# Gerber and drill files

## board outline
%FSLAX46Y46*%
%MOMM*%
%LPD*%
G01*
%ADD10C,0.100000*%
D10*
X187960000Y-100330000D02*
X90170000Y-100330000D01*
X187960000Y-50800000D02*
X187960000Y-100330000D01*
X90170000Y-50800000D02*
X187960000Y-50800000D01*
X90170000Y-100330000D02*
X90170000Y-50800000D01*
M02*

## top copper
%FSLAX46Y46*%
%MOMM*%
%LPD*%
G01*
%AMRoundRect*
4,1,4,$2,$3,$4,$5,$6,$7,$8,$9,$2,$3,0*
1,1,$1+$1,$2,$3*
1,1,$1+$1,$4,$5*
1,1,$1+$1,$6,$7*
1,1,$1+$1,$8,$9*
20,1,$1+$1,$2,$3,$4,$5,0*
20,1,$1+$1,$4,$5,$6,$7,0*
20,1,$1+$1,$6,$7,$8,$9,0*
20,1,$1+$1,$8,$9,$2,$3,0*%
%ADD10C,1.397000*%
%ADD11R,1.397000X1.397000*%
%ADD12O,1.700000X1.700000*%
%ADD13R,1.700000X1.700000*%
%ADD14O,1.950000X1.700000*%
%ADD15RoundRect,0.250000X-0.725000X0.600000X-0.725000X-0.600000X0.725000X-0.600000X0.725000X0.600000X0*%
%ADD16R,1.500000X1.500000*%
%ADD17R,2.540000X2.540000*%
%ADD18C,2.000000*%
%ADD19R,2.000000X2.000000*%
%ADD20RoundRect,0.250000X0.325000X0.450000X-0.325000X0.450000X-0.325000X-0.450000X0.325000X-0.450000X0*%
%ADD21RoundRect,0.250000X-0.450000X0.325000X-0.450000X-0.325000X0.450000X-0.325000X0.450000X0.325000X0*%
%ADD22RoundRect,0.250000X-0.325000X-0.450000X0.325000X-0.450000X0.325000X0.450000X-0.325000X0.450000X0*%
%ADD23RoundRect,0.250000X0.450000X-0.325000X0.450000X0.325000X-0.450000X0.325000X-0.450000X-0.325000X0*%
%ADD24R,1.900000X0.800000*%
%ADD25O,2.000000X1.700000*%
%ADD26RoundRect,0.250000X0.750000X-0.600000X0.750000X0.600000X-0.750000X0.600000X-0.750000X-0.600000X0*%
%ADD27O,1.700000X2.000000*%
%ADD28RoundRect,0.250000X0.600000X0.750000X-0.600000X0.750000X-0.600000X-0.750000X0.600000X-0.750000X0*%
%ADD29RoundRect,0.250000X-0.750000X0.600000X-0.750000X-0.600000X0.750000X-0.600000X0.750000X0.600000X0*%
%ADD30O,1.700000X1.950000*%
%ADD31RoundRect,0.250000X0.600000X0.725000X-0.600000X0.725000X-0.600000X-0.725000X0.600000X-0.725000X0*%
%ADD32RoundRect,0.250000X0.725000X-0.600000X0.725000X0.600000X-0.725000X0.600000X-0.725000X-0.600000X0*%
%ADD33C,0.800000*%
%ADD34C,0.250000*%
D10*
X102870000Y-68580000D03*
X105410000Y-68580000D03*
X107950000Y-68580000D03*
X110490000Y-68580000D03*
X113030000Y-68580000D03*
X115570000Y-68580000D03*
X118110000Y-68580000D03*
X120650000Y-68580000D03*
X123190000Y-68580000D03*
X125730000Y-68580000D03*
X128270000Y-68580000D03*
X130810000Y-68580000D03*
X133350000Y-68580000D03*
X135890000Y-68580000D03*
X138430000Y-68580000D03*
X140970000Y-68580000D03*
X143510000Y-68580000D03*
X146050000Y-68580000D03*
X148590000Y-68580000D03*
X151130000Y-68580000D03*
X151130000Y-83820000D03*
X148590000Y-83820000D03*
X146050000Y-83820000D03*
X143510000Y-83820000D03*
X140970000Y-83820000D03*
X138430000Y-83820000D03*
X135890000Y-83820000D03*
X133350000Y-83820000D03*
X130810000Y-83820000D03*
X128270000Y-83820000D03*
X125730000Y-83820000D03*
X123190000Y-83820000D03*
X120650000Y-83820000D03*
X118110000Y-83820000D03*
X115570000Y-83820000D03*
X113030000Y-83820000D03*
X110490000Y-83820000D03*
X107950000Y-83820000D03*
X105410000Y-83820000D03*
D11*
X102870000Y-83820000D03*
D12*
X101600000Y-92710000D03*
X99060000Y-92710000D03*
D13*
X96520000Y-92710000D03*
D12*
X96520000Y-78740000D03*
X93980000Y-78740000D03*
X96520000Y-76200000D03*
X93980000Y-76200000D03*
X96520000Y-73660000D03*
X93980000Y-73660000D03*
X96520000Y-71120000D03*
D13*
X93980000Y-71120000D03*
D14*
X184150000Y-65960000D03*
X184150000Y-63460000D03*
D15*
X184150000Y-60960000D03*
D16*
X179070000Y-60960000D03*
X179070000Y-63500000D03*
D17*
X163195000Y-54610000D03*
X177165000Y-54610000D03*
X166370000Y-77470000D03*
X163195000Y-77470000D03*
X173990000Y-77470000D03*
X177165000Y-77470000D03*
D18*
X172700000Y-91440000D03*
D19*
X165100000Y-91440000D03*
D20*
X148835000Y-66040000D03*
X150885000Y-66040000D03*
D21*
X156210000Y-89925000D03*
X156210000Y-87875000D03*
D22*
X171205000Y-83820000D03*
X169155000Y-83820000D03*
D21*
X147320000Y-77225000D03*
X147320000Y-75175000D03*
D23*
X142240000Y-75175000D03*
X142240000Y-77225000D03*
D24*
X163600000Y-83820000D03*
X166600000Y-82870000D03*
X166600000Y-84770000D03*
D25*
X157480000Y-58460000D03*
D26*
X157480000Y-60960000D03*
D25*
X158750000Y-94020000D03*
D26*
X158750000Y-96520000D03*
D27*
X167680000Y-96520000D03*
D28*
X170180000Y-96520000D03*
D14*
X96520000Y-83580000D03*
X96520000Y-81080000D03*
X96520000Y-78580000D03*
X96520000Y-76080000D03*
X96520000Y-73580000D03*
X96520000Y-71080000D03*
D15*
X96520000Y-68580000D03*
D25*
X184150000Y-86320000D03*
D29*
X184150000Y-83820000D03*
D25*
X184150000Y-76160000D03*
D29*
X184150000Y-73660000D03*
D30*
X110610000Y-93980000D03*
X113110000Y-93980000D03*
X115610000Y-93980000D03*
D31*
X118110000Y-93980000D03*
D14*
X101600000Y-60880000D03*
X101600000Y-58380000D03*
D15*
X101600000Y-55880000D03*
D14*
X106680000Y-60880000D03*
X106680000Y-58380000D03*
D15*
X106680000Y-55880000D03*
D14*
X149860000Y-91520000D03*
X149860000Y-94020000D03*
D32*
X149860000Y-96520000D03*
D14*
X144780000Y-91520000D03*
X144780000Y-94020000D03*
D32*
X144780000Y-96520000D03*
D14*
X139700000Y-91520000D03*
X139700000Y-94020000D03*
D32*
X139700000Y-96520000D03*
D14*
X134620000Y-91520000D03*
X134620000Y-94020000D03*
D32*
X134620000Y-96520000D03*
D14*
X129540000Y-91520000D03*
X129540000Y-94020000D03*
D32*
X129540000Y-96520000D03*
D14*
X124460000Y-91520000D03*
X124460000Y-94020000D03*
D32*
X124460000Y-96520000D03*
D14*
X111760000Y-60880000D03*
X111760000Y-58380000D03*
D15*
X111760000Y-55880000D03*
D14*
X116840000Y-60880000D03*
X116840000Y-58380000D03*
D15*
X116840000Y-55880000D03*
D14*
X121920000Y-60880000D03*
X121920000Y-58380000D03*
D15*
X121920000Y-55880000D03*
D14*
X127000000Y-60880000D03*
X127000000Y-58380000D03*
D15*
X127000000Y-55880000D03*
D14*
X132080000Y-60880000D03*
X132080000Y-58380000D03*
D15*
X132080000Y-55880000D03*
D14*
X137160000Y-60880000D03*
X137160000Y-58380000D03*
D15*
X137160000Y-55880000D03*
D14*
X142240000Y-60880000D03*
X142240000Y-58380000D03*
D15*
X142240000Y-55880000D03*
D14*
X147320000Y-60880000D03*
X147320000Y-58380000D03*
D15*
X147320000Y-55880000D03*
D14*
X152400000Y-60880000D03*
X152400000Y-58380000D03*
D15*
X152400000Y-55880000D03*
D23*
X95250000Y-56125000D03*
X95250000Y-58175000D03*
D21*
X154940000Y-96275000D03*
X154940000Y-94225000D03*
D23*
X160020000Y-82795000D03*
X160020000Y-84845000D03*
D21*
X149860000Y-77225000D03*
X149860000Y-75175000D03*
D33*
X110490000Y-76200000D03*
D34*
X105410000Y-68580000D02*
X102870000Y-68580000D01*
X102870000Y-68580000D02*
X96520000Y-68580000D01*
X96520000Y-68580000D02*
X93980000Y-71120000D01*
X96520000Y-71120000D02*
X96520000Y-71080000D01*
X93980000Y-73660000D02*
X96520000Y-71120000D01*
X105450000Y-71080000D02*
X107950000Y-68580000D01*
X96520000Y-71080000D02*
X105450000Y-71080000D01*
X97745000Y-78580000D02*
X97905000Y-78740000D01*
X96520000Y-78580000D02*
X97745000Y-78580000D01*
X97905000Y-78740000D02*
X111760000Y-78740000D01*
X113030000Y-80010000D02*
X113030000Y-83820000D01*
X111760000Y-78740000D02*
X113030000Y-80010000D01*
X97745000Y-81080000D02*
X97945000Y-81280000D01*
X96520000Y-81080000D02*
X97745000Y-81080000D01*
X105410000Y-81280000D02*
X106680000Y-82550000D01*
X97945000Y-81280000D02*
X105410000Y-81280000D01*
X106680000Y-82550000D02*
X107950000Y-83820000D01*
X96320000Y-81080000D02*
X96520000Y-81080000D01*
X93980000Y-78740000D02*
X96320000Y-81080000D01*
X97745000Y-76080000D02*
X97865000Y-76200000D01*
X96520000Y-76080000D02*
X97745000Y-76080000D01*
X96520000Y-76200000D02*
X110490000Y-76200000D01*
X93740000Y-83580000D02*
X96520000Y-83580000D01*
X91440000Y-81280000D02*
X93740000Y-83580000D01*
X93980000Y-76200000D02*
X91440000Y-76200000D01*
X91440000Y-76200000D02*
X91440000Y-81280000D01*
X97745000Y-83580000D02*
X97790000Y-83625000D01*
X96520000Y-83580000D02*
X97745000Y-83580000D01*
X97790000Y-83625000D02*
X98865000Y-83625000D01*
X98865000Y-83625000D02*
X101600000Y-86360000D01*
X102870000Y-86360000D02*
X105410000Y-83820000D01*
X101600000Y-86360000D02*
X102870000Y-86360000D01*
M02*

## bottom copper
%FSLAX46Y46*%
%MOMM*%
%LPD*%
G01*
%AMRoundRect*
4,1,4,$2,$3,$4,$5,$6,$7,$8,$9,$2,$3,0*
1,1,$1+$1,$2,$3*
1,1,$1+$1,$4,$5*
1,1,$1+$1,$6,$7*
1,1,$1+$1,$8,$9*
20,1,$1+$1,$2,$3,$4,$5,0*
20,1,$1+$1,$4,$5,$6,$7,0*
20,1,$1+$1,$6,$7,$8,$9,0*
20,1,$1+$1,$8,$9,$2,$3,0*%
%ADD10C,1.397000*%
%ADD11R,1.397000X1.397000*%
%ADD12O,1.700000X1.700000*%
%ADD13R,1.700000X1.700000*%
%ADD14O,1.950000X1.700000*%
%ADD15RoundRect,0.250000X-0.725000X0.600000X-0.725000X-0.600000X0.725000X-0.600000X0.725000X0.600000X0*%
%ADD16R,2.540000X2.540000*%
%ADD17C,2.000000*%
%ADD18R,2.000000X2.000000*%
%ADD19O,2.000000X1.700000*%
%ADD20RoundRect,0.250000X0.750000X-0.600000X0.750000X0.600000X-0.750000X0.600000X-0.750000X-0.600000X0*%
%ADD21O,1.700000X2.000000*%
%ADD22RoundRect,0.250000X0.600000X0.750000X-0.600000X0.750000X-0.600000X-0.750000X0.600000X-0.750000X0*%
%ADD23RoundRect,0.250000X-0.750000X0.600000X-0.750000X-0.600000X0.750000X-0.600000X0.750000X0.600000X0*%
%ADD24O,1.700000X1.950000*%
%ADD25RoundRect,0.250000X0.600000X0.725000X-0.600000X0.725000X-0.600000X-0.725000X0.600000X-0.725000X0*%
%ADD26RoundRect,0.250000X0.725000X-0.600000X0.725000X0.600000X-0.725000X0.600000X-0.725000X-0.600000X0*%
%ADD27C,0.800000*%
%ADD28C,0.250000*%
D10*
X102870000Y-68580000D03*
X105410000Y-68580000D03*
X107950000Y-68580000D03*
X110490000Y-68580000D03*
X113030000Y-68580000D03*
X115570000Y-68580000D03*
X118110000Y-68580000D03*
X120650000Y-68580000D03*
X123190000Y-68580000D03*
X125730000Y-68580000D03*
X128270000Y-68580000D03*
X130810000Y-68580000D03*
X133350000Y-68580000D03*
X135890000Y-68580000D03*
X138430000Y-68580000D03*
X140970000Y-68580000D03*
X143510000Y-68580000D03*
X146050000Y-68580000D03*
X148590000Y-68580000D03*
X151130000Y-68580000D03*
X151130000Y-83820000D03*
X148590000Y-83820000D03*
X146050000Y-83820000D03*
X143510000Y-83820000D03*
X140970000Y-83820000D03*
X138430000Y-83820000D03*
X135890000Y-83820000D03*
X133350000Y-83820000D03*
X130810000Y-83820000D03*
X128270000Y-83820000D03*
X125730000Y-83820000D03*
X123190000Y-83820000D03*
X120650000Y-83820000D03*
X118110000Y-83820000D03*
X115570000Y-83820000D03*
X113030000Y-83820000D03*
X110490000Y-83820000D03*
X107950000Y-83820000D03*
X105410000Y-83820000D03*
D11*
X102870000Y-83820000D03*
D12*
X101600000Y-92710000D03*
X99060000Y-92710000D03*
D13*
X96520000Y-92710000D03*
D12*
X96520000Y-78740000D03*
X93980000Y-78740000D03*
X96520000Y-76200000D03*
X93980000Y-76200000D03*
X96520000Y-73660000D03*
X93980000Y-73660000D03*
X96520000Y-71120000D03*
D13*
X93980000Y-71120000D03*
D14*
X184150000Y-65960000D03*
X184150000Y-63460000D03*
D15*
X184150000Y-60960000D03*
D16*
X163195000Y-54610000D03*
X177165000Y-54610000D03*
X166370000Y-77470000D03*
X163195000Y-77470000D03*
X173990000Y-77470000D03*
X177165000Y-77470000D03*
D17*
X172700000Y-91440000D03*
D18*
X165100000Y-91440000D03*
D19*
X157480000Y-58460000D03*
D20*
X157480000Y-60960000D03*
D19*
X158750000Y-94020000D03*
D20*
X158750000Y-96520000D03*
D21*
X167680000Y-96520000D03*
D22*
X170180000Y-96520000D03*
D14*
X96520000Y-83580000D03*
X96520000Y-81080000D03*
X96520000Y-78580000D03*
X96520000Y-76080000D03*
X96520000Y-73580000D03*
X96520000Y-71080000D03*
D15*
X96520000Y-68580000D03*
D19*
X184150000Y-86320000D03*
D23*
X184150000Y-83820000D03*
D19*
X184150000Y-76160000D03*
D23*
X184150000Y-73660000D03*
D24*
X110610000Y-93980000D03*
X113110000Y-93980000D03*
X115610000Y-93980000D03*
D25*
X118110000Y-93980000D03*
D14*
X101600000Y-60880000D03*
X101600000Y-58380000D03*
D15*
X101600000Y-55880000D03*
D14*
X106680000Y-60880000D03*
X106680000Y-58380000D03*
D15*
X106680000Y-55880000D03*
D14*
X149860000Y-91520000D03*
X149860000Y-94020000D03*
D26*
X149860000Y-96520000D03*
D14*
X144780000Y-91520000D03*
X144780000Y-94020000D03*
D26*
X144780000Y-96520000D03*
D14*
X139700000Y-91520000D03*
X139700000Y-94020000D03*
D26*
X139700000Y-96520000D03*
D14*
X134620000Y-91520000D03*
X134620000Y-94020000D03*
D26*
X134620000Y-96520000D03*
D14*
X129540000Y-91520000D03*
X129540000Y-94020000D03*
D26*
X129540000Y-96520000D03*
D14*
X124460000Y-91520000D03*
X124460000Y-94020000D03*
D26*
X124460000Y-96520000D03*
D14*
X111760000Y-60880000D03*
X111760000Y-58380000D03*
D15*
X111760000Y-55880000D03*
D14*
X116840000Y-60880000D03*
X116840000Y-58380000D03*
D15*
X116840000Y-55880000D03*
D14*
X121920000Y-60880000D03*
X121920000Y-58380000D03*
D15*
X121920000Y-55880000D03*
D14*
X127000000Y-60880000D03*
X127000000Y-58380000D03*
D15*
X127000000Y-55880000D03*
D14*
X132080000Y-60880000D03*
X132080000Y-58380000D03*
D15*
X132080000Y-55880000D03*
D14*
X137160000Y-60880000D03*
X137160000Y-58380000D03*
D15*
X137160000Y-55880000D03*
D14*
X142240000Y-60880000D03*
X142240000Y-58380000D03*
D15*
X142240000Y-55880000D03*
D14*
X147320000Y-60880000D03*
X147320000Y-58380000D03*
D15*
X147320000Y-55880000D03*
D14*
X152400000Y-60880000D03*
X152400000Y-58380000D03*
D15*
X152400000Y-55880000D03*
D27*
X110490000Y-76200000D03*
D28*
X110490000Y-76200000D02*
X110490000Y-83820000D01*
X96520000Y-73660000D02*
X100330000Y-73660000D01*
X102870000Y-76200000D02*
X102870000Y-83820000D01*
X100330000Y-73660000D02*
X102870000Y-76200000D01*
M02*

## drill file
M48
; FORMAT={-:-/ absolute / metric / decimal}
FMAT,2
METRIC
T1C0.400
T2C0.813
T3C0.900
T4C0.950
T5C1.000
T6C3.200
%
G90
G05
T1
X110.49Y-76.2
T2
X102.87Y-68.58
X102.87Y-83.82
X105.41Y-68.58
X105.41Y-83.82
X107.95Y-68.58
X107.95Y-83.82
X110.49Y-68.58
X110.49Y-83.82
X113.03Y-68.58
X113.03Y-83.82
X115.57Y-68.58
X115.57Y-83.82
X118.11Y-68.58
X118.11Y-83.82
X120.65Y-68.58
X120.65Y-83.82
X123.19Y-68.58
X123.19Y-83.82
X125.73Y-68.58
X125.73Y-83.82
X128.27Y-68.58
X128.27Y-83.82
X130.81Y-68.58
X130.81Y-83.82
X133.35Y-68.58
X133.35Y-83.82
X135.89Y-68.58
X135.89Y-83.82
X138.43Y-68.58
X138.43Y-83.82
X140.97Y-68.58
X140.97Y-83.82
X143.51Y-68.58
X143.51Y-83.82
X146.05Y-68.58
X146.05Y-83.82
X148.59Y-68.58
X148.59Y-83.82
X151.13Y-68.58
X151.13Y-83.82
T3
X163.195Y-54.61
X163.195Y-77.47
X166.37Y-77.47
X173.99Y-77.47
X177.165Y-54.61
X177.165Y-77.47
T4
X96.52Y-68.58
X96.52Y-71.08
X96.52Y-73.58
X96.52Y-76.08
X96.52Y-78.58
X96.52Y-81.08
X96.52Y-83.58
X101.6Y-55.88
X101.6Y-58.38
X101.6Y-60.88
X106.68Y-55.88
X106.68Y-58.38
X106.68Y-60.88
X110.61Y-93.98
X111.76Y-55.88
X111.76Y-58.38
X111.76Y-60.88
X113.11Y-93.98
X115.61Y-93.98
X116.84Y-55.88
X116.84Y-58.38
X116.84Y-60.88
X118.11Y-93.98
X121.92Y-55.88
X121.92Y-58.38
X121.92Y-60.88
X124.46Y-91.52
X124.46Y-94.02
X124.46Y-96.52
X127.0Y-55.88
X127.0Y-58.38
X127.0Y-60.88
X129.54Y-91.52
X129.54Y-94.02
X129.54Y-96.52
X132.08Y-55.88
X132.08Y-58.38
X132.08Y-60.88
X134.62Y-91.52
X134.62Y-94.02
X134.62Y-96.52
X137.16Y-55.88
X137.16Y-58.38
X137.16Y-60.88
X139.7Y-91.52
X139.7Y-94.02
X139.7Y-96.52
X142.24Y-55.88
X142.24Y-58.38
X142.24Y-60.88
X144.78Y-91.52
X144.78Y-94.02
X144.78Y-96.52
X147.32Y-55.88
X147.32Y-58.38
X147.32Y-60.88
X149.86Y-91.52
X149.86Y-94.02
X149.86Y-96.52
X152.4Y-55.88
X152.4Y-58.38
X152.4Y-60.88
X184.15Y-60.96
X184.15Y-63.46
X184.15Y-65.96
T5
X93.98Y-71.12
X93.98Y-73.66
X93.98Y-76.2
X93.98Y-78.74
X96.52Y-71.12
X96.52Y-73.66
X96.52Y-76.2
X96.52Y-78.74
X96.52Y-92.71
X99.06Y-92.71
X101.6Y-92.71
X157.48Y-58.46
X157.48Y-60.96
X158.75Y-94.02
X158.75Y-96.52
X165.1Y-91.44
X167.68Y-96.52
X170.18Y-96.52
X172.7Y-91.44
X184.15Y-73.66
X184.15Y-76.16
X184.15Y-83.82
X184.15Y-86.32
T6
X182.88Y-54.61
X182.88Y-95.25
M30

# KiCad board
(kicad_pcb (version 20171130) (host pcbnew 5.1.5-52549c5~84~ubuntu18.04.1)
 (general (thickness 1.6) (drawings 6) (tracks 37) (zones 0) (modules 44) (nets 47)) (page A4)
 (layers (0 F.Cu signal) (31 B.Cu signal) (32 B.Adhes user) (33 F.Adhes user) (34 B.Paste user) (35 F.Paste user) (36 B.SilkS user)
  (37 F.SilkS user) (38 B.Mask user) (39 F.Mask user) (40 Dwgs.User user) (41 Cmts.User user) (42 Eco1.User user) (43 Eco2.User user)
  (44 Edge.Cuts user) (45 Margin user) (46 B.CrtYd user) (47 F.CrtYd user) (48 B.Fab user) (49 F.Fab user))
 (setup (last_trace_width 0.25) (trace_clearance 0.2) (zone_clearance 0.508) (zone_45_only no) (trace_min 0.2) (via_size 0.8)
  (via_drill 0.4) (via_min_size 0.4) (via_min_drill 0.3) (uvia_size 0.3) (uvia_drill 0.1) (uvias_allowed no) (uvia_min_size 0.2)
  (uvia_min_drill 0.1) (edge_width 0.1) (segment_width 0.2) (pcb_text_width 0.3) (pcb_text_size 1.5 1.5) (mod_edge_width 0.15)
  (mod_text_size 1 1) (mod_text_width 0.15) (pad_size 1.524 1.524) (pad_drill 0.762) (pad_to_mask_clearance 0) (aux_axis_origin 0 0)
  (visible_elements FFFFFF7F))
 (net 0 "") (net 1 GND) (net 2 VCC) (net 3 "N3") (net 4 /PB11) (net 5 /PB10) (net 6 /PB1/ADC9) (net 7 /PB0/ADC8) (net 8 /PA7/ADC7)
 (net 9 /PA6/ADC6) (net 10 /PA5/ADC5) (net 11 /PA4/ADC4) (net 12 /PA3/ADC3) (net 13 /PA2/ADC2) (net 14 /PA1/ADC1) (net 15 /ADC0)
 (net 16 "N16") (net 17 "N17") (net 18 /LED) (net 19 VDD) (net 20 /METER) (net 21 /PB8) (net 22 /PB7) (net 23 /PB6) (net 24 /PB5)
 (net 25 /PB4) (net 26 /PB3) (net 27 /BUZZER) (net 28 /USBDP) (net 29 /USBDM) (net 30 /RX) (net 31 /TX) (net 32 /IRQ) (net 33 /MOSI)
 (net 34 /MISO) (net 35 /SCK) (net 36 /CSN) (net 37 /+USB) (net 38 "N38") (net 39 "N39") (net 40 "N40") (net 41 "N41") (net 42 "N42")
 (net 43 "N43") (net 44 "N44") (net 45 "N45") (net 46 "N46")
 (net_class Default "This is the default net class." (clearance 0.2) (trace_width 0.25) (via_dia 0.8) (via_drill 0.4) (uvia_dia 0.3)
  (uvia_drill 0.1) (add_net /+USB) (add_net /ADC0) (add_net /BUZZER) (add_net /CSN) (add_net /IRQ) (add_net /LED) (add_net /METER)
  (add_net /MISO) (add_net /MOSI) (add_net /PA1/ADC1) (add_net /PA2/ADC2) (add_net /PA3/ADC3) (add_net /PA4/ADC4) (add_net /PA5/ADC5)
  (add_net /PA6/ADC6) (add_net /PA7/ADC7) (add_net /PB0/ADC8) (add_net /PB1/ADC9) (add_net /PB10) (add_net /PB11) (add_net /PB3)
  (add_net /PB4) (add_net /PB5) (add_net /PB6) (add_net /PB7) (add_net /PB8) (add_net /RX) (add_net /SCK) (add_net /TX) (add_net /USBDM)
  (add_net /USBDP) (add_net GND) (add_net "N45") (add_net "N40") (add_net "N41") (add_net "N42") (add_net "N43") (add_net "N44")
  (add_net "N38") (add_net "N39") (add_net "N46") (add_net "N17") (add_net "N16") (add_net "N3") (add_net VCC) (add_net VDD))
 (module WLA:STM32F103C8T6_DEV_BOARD (layer F.Cu) (at 127 76.2)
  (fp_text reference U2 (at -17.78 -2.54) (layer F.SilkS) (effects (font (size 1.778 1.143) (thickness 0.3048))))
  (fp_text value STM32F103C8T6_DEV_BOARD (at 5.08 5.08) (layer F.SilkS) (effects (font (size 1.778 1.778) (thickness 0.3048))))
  (pad 40 thru_hole circle (at -24.13 -7.62) (size 1.397 1.397) (drill 0.8128) (layers *.Cu *.Mask) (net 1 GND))
  (pad 39 thru_hole circle (at -21.59 -7.62) (size 1.397 1.397) (drill 0.8128) (layers *.Cu *.Mask) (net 1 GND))
  (pad 38 thru_hole circle (at -19.05 -7.62) (size 1.397 1.397) (drill 0.8128) (layers *.Cu *.Mask) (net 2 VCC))
  (pad 37 thru_hole circle (at -16.51 -7.62) (size 1.397 1.397) (drill 0.8128) (layers *.Cu *.Mask) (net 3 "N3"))
  (pad 36 thru_hole circle (at -13.97 -7.62) (size 1.397 1.397) (drill 0.8128) (layers *.Cu *.Mask) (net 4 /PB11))
  (pad 35 thru_hole circle (at -11.43 -7.62) (size 1.397 1.397) (drill 0.8128) (layers *.Cu *.Mask) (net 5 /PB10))
  (pad 34 thru_hole circle (at -8.89 -7.62) (size 1.397 1.397) (drill 0.8128) (layers *.Cu *.Mask) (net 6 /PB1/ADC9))
  (pad 33 thru_hole circle (at -6.35 -7.62) (size 1.397 1.397) (drill 0.8128) (layers *.Cu *.Mask) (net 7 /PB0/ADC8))
  (pad 32 thru_hole circle (at -3.81 -7.62) (size 1.397 1.397) (drill 0.8128) (layers *.Cu *.Mask) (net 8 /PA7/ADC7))
  (pad 31 thru_hole circle (at -1.27 -7.62) (size 1.397 1.397) (drill 0.8128) (layers *.Cu *.Mask) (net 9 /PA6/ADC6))
  (pad 30 thru_hole circle (at 1.27 -7.62) (size 1.397 1.397) (drill 0.8128) (layers *.Cu *.Mask) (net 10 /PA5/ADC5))
  (pad 29 thru_hole circle (at 3.81 -7.62) (size 1.397 1.397) (drill 0.8128) (layers *.Cu *.Mask) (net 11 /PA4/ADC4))
  (pad 28 thru_hole circle (at 6.35 -7.62) (size 1.397 1.397) (drill 0.8128) (layers *.Cu *.Mask) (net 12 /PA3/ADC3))
  (pad 27 thru_hole circle (at 8.89 -7.62) (size 1.397 1.397) (drill 0.8128) (layers *.Cu *.Mask) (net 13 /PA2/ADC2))
  (pad 26 thru_hole circle (at 11.43 -7.62) (size 1.397 1.397) (drill 0.8128) (layers *.Cu *.Mask) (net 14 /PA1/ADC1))
  (pad 25 thru_hole circle (at 13.97 -7.62) (size 1.397 1.397) (drill 0.8128) (layers *.Cu *.Mask) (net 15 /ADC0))
  (pad 24 thru_hole circle (at 16.51 -7.62) (size 1.397 1.397) (drill 0.8128) (layers *.Cu *.Mask) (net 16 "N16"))
  (pad 23 thru_hole circle (at 19.05 -7.62) (size 1.397 1.397) (drill 0.8128) (layers *.Cu *.Mask) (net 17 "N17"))
  (pad 22 thru_hole circle (at 21.59 -7.62) (size 1.397 1.397) (drill 0.8128) (layers *.Cu *.Mask) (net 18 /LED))
  (pad 21 thru_hole circle (at 24.13 -7.62) (size 1.397 1.397) (drill 0.8128) (layers *.Cu *.Mask) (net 2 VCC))
  (pad 20 thru_hole circle (at 24.13 7.62) (size 1.397 1.397) (drill 0.8128) (layers *.Cu *.Mask) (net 2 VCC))
  (pad 19 thru_hole circle (at 21.59 7.62) (size 1.397 1.397) (drill 0.8128) (layers *.Cu *.Mask) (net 1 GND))
  (pad 18 thru_hole circle (at 19.05 7.62) (size 1.397 1.397) (drill 0.8128) (layers *.Cu *.Mask) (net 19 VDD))
  (pad 17 thru_hole circle (at 16.51 7.62) (size 1.397 1.397) (drill 0.8128) (layers *.Cu *.Mask) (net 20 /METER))
  (pad 16 thru_hole circle (at 13.97 7.62) (size 1.397 1.397) (drill 0.8128) (layers *.Cu *.Mask) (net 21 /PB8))
  (pad 15 thru_hole circle (at 11.43 7.62) (size 1.397 1.397) (drill 0.8128) (layers *.Cu *.Mask) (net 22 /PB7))
  (pad 14 thru_hole circle (at 8.89 7.62) (size 1.397 1.397) (drill 0.8128) (layers *.Cu *.Mask) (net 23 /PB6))
  (pad 13 thru_hole circle (at 6.35 7.62) (size 1.397 1.397) (drill 0.8128) (layers *.Cu *.Mask) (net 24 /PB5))
  (pad 12 thru_hole circle (at 3.81 7.62) (size 1.397 1.397) (drill 0.8128) (layers *.Cu *.Mask) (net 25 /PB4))
  (pad 11 thru_hole circle (at 1.27 7.62) (size 1.397 1.397) (drill 0.8128) (layers *.Cu *.Mask) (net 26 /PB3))
  (pad 10 thru_hole circle (at -1.27 7.62) (size 1.397 1.397) (drill 0.8128) (layers *.Cu *.Mask) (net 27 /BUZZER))
  (pad 9 thru_hole circle (at -3.81 7.62) (size 1.397 1.397) (drill 0.8128) (layers *.Cu *.Mask) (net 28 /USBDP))
  (pad 8 thru_hole circle (at -6.35 7.62) (size 1.397 1.397) (drill 0.8128) (layers *.Cu *.Mask) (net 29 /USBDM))
  (pad 7 thru_hole circle (at -8.89 7.62) (size 1.397 1.397) (drill 0.8128) (layers *.Cu *.Mask) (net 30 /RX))
  (pad 6 thru_hole circle (at -11.43 7.62) (size 1.397 1.397) (drill 0.8128) (layers *.Cu *.Mask) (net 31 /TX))
  (pad 5 thru_hole circle (at -13.97 7.62) (size 1.397 1.397) (drill 0.8128) (layers *.Cu *.Mask) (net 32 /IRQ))
  (pad 4 thru_hole circle (at -16.51 7.62) (size 1.397 1.397) (drill 0.8128) (layers *.Cu *.Mask) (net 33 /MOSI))
  (pad 3 thru_hole circle (at -19.05 7.62) (size 1.397 1.397) (drill 0.8128) (layers *.Cu *.Mask) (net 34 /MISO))
  (pad 2 thru_hole circle (at -21.59 7.62) (size 1.397 1.397) (drill 0.8128) (layers *.Cu *.Mask) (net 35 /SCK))
  (pad 1 thru_hole rect (at -24.13 7.62) (size 1.397 1.397) (drill 0.8128) (layers *.Cu *.Mask) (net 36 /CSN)))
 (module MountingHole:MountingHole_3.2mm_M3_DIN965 (layer F.Cu) (at 182.88 95.25)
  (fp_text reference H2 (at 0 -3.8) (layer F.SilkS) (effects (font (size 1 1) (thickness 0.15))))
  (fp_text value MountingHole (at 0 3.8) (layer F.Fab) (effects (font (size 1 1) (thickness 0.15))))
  (pad 1 np_thru_hole circle (at 0 0) (size 3.2 3.2) (drill 3.2) (layers *.Cu *.Mask)))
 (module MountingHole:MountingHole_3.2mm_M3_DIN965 (layer F.Cu) (at 182.88 54.61)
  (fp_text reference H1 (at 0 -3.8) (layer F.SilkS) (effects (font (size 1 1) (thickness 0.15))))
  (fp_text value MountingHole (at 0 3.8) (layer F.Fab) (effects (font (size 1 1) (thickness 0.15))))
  (pad 1 np_thru_hole circle (at 0 0) (size 3.2 3.2) (drill 3.2) (layers *.Cu *.Mask)))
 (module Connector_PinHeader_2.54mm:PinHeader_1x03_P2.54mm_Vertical (layer F.Cu) (at 96.52 92.71 90)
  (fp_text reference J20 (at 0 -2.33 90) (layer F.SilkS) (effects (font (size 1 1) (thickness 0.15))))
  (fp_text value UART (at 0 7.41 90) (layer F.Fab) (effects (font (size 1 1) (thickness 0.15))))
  (pad 3 thru_hole oval (at 0 5.08 90) (size 1.7 1.7) (drill 1) (layers *.Cu *.Mask) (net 30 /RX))
  (pad 2 thru_hole oval (at 0 2.54 90) (size 1.7 1.7) (drill 1) (layers *.Cu *.Mask) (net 31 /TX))
  (pad 1 thru_hole rect (at 0 0 90) (size 1.7 1.7) (drill 1) (layers *.Cu *.Mask) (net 1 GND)))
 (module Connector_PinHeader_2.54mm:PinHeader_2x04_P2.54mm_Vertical (layer F.Cu) (at 93.98 71.12)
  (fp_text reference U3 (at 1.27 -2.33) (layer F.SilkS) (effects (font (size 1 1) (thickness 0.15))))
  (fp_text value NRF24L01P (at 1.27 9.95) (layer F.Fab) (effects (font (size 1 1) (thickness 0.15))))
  (pad 8 thru_hole oval (at 2.54 7.62) (size 1.7 1.7) (drill 1) (layers *.Cu *.Mask) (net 32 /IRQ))
  (pad 7 thru_hole oval (at 0 7.62) (size 1.7 1.7) (drill 1) (layers *.Cu *.Mask) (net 34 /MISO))
  (pad 6 thru_hole oval (at 2.54 5.08) (size 1.7 1.7) (drill 1) (layers *.Cu *.Mask) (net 33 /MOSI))
  (pad 5 thru_hole oval (at 0 5.08) (size 1.7 1.7) (drill 1) (layers *.Cu *.Mask) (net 35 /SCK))
  (pad 4 thru_hole oval (at 2.54 2.54) (size 1.7 1.7) (drill 1) (layers *.Cu *.Mask) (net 36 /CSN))
  (pad 3 thru_hole oval (at 0 2.54) (size 1.7 1.7) (drill 1) (layers *.Cu *.Mask) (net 2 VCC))
  (pad 2 thru_hole oval (at 2.54 0) (size 1.7 1.7) (drill 1) (layers *.Cu *.Mask) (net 2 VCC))
  (pad 1 thru_hole rect (at 0 0) (size 1.7 1.7) (drill 1) (layers *.Cu *.Mask) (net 1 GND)))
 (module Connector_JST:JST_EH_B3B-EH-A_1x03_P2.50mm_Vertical (layer F.Cu) (at 184.15 60.96 270)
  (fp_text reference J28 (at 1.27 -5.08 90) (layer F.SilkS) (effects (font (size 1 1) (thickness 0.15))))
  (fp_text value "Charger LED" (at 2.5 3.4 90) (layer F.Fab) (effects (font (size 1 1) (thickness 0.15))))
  (pad 3 thru_hole oval (at 5 0 270) (size 1.7 1.95) (drill 0.95) (layers *.Cu *.Mask) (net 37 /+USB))
  (pad 2 thru_hole oval (at 2.5 0 270) (size 1.7 1.95) (drill 0.95) (layers *.Cu *.Mask) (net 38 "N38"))
  (pad 1 thru_hole roundrect (at 0 0 270) (size 1.7 1.95) (drill 0.95) (layers *.Cu *.Mask) (roundrect_rratio 0.147059) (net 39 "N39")))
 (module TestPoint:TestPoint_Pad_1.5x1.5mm (layer F.Cu) (at 179.07 60.96 90)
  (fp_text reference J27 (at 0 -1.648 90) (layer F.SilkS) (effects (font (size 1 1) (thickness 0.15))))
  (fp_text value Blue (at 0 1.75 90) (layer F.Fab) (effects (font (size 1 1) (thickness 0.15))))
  (pad 1 smd rect (at 0 0 90) (size 1.5 1.5) (layers F.Cu F.Mask) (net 39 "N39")))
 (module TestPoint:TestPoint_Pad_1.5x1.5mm (layer F.Cu) (at 179.07 63.5 90)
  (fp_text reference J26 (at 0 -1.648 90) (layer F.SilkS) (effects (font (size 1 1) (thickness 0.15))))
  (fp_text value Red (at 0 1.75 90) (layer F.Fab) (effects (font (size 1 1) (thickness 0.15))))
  (pad 1 smd rect (at 0 0 90) (size 1.5 1.5) (layers F.Cu F.Mask) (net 38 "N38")))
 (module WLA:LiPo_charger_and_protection (layer F.Cu) (at 170.18 66.04 270)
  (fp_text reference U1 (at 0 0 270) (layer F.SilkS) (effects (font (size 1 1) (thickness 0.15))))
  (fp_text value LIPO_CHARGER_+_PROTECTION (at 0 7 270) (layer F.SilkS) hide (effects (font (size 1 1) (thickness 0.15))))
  (pad 6 thru_hole rect (at -11.43 6.985 270) (size 2.54 2.54) (drill 0.9) (layers *.Cu *.Mask) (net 1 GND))
  (pad 5 thru_hole rect (at -11.43 -6.985 270) (size 2.54 2.54) (drill 0.9) (layers *.Cu *.Mask) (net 37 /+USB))
  (pad 2 thru_hole rect (at 11.43 3.81 270) (size 2.54 2.54) (drill 0.9) (layers *.Cu *.Mask) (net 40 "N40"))
  (pad 4 thru_hole rect (at 11.43 6.985 270) (size 2.54 2.54) (drill 0.9) (layers *.Cu *.Mask) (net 1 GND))
  (pad 1 thru_hole rect (at 11.43 -3.81 270) (size 2.54 2.54) (drill 0.9) (layers *.Cu *.Mask) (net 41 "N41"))
  (pad 3 thru_hole rect (at 11.43 -6.985 270) (size 2.54 2.54) (drill 0.9) (layers *.Cu *.Mask) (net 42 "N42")))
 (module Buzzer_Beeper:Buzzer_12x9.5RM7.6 (layer F.Cu) (at 165.1 91.44)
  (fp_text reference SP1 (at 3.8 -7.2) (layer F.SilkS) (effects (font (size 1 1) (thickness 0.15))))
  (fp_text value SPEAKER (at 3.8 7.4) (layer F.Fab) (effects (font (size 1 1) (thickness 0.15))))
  (pad 2 thru_hole circle (at 7.6 0) (size 2 2) (drill 1) (layers *.Cu *.Mask) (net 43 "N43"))
  (pad 1 thru_hole rect (at 0 0) (size 2 2) (drill 1) (layers *.Cu *.Mask) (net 19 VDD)))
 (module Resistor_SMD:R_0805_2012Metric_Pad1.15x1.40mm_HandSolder (layer F.Cu) (at 149.86 66.04 180)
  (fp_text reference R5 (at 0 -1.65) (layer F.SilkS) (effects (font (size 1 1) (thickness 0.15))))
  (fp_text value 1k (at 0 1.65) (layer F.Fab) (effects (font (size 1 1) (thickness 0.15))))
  (pad 2 smd roundrect (at 1.025 0 180) (size 1.15 1.4) (layers F.Cu F.Paste F.Mask) (roundrect_rratio 0.217391) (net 18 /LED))
  (pad 1 smd roundrect (at -1.025 0 180) (size 1.15 1.4) (layers F.Cu F.Paste F.Mask) (roundrect_rratio 0.217391) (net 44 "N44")))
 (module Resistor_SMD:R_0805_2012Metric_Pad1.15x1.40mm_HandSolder (layer F.Cu) (at 156.21 88.9 270)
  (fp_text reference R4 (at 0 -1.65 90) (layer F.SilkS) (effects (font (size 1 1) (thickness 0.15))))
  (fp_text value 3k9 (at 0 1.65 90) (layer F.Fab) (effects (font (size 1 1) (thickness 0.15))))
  (pad 2 smd roundrect (at 1.025 0 270) (size 1.15 1.4) (layers F.Cu F.Paste F.Mask) (roundrect_rratio 0.217391) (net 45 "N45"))
  (pad 1 smd roundrect (at -1.025 0 270) (size 1.15 1.4) (layers F.Cu F.Paste F.Mask) (roundrect_rratio 0.217391) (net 20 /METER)))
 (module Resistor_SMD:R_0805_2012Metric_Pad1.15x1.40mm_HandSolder (layer F.Cu) (at 170.18 83.82)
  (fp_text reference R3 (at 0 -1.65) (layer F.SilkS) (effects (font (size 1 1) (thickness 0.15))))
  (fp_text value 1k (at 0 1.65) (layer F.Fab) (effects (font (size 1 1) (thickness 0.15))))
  (pad 2 smd roundrect (at 1.025 0) (size 1.15 1.4) (layers F.Cu F.Paste F.Mask) (roundrect_rratio 0.217391) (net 27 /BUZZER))
  (pad 1 smd roundrect (at -1.025 0) (size 1.15 1.4) (layers F.Cu F.Paste F.Mask) (roundrect_rratio 0.217391) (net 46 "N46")))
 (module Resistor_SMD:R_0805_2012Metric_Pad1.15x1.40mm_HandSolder (layer F.Cu) (at 147.32 76.2 270)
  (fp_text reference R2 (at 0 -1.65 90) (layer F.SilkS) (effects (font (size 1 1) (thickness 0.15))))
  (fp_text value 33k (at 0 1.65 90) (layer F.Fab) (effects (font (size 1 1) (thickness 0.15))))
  (pad 2 smd roundrect (at 1.025 0 270) (size 1.15 1.4) (layers F.Cu F.Paste F.Mask) (roundrect_rratio 0.217391) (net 1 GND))
  (pad 1 smd roundrect (at -1.025 0 270) (size 1.15 1.4) (layers F.Cu F.Paste F.Mask) (roundrect_rratio 0.217391) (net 15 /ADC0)))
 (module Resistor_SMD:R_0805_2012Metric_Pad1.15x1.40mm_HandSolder (layer F.Cu) (at 142.24 76.2 90)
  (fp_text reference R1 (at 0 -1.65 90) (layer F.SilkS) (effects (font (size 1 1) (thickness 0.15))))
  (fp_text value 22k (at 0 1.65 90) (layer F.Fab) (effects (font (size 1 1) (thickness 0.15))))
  (pad 2 smd roundrect (at 1.025 0 90) (size 1.15 1.4) (layers F.Cu F.Paste F.Mask) (roundrect_rratio 0.217391) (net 15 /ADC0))
  (pad 1 smd roundrect (at -1.025 0 90) (size 1.15 1.4) (layers F.Cu F.Paste F.Mask) (roundrect_rratio 0.217391) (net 19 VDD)))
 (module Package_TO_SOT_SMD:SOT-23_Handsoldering (layer F.Cu) (at 165.1 83.82 180)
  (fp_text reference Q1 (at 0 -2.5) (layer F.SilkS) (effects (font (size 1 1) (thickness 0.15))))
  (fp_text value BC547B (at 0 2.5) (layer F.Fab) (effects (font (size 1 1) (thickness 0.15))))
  (pad 3 smd rect (at 1.5 0 180) (size 1.9 0.8) (layers F.Cu F.Paste F.Mask) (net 1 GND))
  (pad 2 smd rect (at -1.5 0.95 180) (size 1.9 0.8) (layers F.Cu F.Paste F.Mask) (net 46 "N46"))
  (pad 1 smd rect (at -1.5 -0.95 180) (size 1.9 0.8) (layers F.Cu F.Paste F.Mask) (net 43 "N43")))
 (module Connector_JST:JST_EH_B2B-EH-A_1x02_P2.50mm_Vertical (layer F.Cu) (at 157.48 60.96 90)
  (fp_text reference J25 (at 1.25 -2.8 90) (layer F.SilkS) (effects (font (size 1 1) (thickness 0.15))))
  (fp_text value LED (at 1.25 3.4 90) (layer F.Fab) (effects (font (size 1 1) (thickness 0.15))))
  (pad 2 thru_hole oval (at 2.5 0 90) (size 1.7 2) (drill 1) (layers *.Cu *.Mask) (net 2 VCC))
  (pad 1 thru_hole roundrect (at 0 0 90) (size 1.7 2) (drill 1) (layers *.Cu *.Mask) (roundrect_rratio 0.147059) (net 44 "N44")))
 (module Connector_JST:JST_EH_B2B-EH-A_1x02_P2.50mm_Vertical (layer F.Cu) (at 158.75 96.52 90)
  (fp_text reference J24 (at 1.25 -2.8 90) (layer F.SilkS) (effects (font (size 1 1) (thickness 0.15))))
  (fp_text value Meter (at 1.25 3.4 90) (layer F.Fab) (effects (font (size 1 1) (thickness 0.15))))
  (pad 2 thru_hole oval (at 2.5 0 90) (size 1.7 2) (drill 1) (layers *.Cu *.Mask) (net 45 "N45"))
  (pad 1 thru_hole roundrect (at 0 0 90) (size 1.7 2) (drill 1) (layers *.Cu *.Mask) (roundrect_rratio 0.147059) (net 1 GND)))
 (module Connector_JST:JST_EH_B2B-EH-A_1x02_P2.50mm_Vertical (layer F.Cu) (at 170.18 96.52 180)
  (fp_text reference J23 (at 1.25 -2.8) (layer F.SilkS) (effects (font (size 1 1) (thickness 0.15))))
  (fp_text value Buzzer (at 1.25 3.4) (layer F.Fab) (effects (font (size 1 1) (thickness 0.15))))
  (pad 2 thru_hole oval (at 2.5 0 180) (size 1.7 2) (drill 1) (layers *.Cu *.Mask) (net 19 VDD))
  (pad 1 thru_hole roundrect (at 0 0 180) (size 1.7 2) (drill 1) (layers *.Cu *.Mask) (roundrect_rratio 0.147059) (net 43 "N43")))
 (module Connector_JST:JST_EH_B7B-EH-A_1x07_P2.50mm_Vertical (layer F.Cu) (at 96.52 68.58 270)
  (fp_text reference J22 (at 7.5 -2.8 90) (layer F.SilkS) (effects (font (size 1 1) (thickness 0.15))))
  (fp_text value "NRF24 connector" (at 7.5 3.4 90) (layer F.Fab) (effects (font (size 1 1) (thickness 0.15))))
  (pad 7 thru_hole oval (at 15 0 270) (size 1.7 1.95) (drill 0.95) (layers *.Cu *.Mask) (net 35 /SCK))
  (pad 6 thru_hole oval (at 12.5 0 270) (size 1.7 1.95) (drill 0.95) (layers *.Cu *.Mask) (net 34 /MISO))
  (pad 5 thru_hole oval (at 10 0 270) (size 1.7 1.95) (drill 0.95) (layers *.Cu *.Mask) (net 32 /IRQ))
  (pad 4 thru_hole oval (at 7.5 0 270) (size 1.7 1.95) (drill 0.95) (layers *.Cu *.Mask) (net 33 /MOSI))
  (pad 3 thru_hole oval (at 5 0 270) (size 1.7 1.95) (drill 0.95) (layers *.Cu *.Mask) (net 36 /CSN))
  (pad 2 thru_hole oval (at 2.5 0 270) (size 1.7 1.95) (drill 0.95) (layers *.Cu *.Mask) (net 2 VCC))
  (pad 1 thru_hole roundrect (at 0 0 270) (size 1.7 1.95) (drill 0.95) (layers *.Cu *.Mask) (roundrect_rratio 0.147059) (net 1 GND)))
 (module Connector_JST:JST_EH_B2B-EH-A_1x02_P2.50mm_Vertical (layer F.Cu) (at 184.15 83.82 270)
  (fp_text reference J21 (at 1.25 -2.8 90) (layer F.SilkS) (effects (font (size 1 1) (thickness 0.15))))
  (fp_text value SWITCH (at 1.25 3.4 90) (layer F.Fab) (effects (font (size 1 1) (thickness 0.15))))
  (pad 2 thru_hole oval (at 2.5 0 270) (size 1.7 2) (drill 1) (layers *.Cu *.Mask) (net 19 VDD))
  (pad 1 thru_hole roundrect (at 0 0 270) (size 1.7 2) (drill 1) (layers *.Cu *.Mask) (roundrect_rratio 0.147059) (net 42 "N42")))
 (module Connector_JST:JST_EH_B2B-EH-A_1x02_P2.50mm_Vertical (layer F.Cu) (at 184.15 73.66 270)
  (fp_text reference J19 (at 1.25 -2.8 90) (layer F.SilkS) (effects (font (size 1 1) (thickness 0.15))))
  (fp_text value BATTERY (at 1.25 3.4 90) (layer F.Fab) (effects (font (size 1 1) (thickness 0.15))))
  (pad 2 thru_hole oval (at 2.5 0 270) (size 1.7 2) (drill 1) (layers *.Cu *.Mask) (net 41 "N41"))
  (pad 1 thru_hole roundrect (at 0 0 270) (size 1.7 2) (drill 1) (layers *.Cu *.Mask) (roundrect_rratio 0.147059) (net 40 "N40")))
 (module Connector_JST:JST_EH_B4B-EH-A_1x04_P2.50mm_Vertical (layer F.Cu) (at 118.11 93.98 180)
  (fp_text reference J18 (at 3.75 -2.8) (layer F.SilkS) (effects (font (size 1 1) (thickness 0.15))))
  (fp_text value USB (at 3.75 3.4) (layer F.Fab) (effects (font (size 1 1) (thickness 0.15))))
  (pad 4 thru_hole oval (at 7.5 0 180) (size 1.7 1.95) (drill 0.95) (layers *.Cu *.Mask) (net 37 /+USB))
  (pad 3 thru_hole oval (at 5 0 180) (size 1.7 1.95) (drill 0.95) (layers *.Cu *.Mask) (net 29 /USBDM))
  (pad 2 thru_hole oval (at 2.5 0 180) (size 1.7 1.95) (drill 0.95) (layers *.Cu *.Mask) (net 28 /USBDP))
  (pad 1 thru_hole roundrect (at 0 0 180) (size 1.7 1.95) (drill 0.95) (layers *.Cu *.Mask) (roundrect_rratio 0.147059) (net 1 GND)))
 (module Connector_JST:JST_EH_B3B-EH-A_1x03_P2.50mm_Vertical (layer F.Cu) (at 101.6 55.88 270)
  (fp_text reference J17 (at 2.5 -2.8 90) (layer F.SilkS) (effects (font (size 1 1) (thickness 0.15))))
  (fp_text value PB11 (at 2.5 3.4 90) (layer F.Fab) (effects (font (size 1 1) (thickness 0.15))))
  (pad 3 thru_hole oval (at 5 0 270) (size 1.7 1.95) (drill 0.95) (layers *.Cu *.Mask) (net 4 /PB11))
  (pad 2 thru_hole oval (at 2.5 0 270) (size 1.7 1.95) (drill 0.95) (layers *.Cu *.Mask) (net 2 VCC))
  (pad 1 thru_hole roundrect (at 0 0 270) (size 1.7 1.95) (drill 0.95) (layers *.Cu *.Mask) (roundrect_rratio 0.147059) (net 1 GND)))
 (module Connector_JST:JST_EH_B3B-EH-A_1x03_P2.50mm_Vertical (layer F.Cu) (at 106.68 55.88 270)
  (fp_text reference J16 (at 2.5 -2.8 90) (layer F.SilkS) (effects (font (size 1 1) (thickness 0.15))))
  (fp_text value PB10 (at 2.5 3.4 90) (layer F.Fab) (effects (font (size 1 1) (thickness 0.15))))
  (pad 3 thru_hole oval (at 5 0 270) (size 1.7 1.95) (drill 0.95) (layers *.Cu *.Mask) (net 5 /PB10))
  (pad 2 thru_hole oval (at 2.5 0 270) (size 1.7 1.95) (drill 0.95) (layers *.Cu *.Mask) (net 2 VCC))
  (pad 1 thru_hole roundrect (at 0 0 270) (size 1.7 1.95) (drill 0.95) (layers *.Cu *.Mask) (roundrect_rratio 0.147059) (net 1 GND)))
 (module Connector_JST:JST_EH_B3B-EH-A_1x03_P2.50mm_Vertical (layer F.Cu) (at 149.86 96.52 90)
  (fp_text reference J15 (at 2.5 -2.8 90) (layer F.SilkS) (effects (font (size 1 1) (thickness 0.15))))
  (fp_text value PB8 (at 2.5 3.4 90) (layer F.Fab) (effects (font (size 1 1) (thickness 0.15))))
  (pad 3 thru_hole oval (at 5 0 90) (size 1.7 1.95) (drill 0.95) (layers *.Cu *.Mask) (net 21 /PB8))
  (pad 2 thru_hole oval (at 2.5 0 90) (size 1.7 1.95) (drill 0.95) (layers *.Cu *.Mask) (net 2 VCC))
  (pad 1 thru_hole roundrect (at 0 0 90) (size 1.7 1.95) (drill 0.95) (layers *.Cu *.Mask) (roundrect_rratio 0.147059) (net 1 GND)))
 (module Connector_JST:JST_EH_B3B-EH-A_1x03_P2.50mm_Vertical (layer F.Cu) (at 144.78 96.52 90)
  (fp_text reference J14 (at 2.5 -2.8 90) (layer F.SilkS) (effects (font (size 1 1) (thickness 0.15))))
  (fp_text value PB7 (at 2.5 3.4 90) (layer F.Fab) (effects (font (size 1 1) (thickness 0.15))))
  (pad 3 thru_hole oval (at 5 0 90) (size 1.7 1.95) (drill 0.95) (layers *.Cu *.Mask) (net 22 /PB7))
  (pad 2 thru_hole oval (at 2.5 0 90) (size 1.7 1.95) (drill 0.95) (layers *.Cu *.Mask) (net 2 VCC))
  (pad 1 thru_hole roundrect (at 0 0 90) (size 1.7 1.95) (drill 0.95) (layers *.Cu *.Mask) (roundrect_rratio 0.147059) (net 1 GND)))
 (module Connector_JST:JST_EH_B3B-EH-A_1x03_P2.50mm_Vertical (layer F.Cu) (at 139.7 96.52 90)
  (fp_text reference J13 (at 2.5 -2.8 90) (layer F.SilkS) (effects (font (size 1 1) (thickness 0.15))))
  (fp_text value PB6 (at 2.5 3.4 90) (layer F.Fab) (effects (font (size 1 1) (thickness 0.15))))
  (pad 3 thru_hole oval (at 5 0 90) (size 1.7 1.95) (drill 0.95) (layers *.Cu *.Mask) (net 23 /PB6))
  (pad 2 thru_hole oval (at 2.5 0 90) (size 1.7 1.95) (drill 0.95) (layers *.Cu *.Mask) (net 2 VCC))
  (pad 1 thru_hole roundrect (at 0 0 90) (size 1.7 1.95) (drill 0.95) (layers *.Cu *.Mask) (roundrect_rratio 0.147059) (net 1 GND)))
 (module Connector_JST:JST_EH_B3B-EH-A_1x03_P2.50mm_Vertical (layer F.Cu) (at 134.62 96.52 90)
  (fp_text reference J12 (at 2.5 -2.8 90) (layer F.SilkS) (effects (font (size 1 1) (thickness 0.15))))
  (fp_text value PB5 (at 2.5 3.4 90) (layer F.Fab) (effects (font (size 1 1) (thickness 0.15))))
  (pad 3 thru_hole oval (at 5 0 90) (size 1.7 1.95) (drill 0.95) (layers *.Cu *.Mask) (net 24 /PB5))
  (pad 2 thru_hole oval (at 2.5 0 90) (size 1.7 1.95) (drill 0.95) (layers *.Cu *.Mask) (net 2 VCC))
  (pad 1 thru_hole roundrect (at 0 0 90) (size 1.7 1.95) (drill 0.95) (layers *.Cu *.Mask) (roundrect_rratio 0.147059) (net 1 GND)))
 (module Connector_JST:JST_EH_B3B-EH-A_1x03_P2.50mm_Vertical (layer F.Cu) (at 129.54 96.52 90)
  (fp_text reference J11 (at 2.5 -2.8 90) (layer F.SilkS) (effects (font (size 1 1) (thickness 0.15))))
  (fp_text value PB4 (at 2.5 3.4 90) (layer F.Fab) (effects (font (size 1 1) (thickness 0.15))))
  (pad 3 thru_hole oval (at 5 0 90) (size 1.7 1.95) (drill 0.95) (layers *.Cu *.Mask) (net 25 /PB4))
  (pad 2 thru_hole oval (at 2.5 0 90) (size 1.7 1.95) (drill 0.95) (layers *.Cu *.Mask) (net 2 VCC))
  (pad 1 thru_hole roundrect (at 0 0 90) (size 1.7 1.95) (drill 0.95) (layers *.Cu *.Mask) (roundrect_rratio 0.147059) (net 1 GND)))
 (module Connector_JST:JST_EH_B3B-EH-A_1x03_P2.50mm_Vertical (layer F.Cu) (at 124.46 96.52 90)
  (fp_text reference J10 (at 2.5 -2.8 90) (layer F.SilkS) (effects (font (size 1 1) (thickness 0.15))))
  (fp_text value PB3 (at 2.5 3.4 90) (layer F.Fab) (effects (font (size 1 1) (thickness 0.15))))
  (pad 3 thru_hole oval (at 5 0 90) (size 1.7 1.95) (drill 0.95) (layers *.Cu *.Mask) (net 26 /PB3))
  (pad 2 thru_hole oval (at 2.5 0 90) (size 1.7 1.95) (drill 0.95) (layers *.Cu *.Mask) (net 2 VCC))
  (pad 1 thru_hole roundrect (at 0 0 90) (size 1.7 1.95) (drill 0.95) (layers *.Cu *.Mask) (roundrect_rratio 0.147059) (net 1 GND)))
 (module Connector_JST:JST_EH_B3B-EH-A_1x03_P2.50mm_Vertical (layer F.Cu) (at 111.76 55.88 270)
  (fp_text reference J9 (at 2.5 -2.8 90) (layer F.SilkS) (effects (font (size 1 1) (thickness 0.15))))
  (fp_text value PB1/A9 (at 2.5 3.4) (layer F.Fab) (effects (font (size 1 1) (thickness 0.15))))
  (pad 3 thru_hole oval (at 5 0 270) (size 1.7 1.95) (drill 0.95) (layers *.Cu *.Mask) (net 6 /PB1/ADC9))
  (pad 2 thru_hole oval (at 2.5 0 270) (size 1.7 1.95) (drill 0.95) (layers *.Cu *.Mask) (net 2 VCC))
  (pad 1 thru_hole roundrect (at 0 0 270) (size 1.7 1.95) (drill 0.95) (layers *.Cu *.Mask) (roundrect_rratio 0.147059) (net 1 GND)))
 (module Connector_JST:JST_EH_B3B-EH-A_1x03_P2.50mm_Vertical (layer F.Cu) (at 116.84 55.88 270)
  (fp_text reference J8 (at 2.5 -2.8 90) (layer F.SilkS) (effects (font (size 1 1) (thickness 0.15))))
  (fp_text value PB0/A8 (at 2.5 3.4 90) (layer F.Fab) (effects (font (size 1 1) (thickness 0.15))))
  (pad 3 thru_hole oval (at 5 0 270) (size 1.7 1.95) (drill 0.95) (layers *.Cu *.Mask) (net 7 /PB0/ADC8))
  (pad 2 thru_hole oval (at 2.5 0 270) (size 1.7 1.95) (drill 0.95) (layers *.Cu *.Mask) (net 2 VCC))
  (pad 1 thru_hole roundrect (at 0 0 270) (size 1.7 1.95) (drill 0.95) (layers *.Cu *.Mask) (roundrect_rratio 0.147059) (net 1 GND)))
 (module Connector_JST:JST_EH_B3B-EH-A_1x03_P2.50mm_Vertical (layer F.Cu) (at 121.92 55.88 270)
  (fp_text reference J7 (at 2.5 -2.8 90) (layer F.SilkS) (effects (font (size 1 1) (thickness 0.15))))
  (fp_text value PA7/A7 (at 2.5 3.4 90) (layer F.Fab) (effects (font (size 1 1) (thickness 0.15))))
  (pad 3 thru_hole oval (at 5 0 270) (size 1.7 1.95) (drill 0.95) (layers *.Cu *.Mask) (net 8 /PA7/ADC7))
  (pad 2 thru_hole oval (at 2.5 0 270) (size 1.7 1.95) (drill 0.95) (layers *.Cu *.Mask) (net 2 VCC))
  (pad 1 thru_hole roundrect (at 0 0 270) (size 1.7 1.95) (drill 0.95) (layers *.Cu *.Mask) (roundrect_rratio 0.147059) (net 1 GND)))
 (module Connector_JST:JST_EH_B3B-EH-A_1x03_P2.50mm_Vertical (layer F.Cu) (at 127 55.88 270)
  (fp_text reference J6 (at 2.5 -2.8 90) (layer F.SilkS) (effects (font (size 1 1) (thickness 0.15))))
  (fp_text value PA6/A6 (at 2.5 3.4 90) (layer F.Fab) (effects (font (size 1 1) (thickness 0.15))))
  (pad 3 thru_hole oval (at 5 0 270) (size 1.7 1.95) (drill 0.95) (layers *.Cu *.Mask) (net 9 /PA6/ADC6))
  (pad 2 thru_hole oval (at 2.5 0 270) (size 1.7 1.95) (drill 0.95) (layers *.Cu *.Mask) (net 2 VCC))
  (pad 1 thru_hole roundrect (at 0 0 270) (size 1.7 1.95) (drill 0.95) (layers *.Cu *.Mask) (roundrect_rratio 0.147059) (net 1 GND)))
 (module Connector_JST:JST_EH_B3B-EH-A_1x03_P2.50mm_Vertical (layer F.Cu) (at 132.08 55.88 270)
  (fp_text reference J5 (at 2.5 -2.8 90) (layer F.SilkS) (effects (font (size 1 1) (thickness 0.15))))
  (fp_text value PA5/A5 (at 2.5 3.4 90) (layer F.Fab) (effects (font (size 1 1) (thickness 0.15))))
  (pad 3 thru_hole oval (at 5 0 270) (size 1.7 1.95) (drill 0.95) (layers *.Cu *.Mask) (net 10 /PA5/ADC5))
  (pad 2 thru_hole oval (at 2.5 0 270) (size 1.7 1.95) (drill 0.95) (layers *.Cu *.Mask) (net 2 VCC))
  (pad 1 thru_hole roundrect (at 0 0 270) (size 1.7 1.95) (drill 0.95) (layers *.Cu *.Mask) (roundrect_rratio 0.147059) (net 1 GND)))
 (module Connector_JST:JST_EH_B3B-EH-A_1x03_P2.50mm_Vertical (layer F.Cu) (at 137.16 55.88 270)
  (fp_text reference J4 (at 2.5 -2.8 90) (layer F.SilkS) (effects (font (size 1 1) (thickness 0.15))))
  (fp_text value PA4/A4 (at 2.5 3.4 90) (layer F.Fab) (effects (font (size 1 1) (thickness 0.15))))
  (pad 3 thru_hole oval (at 5 0 270) (size 1.7 1.95) (drill 0.95) (layers *.Cu *.Mask) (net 11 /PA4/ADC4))
  (pad 2 thru_hole oval (at 2.5 0 270) (size 1.7 1.95) (drill 0.95) (layers *.Cu *.Mask) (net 2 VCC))
  (pad 1 thru_hole roundrect (at 0 0 270) (size 1.7 1.95) (drill 0.95) (layers *.Cu *.Mask) (roundrect_rratio 0.147059) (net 1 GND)))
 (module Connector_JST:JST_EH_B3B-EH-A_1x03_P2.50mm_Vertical (layer F.Cu) (at 142.24 55.88 270)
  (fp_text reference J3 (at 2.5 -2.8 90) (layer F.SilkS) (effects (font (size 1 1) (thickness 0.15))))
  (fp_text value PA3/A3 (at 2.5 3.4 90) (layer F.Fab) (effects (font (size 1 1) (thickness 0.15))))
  (pad 3 thru_hole oval (at 5 0 270) (size 1.7 1.95) (drill 0.95) (layers *.Cu *.Mask) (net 12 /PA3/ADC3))
  (pad 2 thru_hole oval (at 2.5 0 270) (size 1.7 1.95) (drill 0.95) (layers *.Cu *.Mask) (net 2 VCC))
  (pad 1 thru_hole roundrect (at 0 0 270) (size 1.7 1.95) (drill 0.95) (layers *.Cu *.Mask) (roundrect_rratio 0.147059) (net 1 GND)))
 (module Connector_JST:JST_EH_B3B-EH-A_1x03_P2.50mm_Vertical (layer F.Cu) (at 147.32 55.88 270)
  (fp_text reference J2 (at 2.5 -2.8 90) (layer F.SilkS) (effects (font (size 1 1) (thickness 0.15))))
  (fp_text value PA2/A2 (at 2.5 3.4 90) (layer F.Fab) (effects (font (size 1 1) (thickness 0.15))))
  (pad 3 thru_hole oval (at 5 0 270) (size 1.7 1.95) (drill 0.95) (layers *.Cu *.Mask) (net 13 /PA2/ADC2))
  (pad 2 thru_hole oval (at 2.5 0 270) (size 1.7 1.95) (drill 0.95) (layers *.Cu *.Mask) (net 2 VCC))
  (pad 1 thru_hole roundrect (at 0 0 270) (size 1.7 1.95) (drill 0.95) (layers *.Cu *.Mask) (roundrect_rratio 0.147059) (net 1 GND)))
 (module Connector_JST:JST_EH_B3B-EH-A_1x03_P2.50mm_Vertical (layer F.Cu) (at 152.4 55.88 270)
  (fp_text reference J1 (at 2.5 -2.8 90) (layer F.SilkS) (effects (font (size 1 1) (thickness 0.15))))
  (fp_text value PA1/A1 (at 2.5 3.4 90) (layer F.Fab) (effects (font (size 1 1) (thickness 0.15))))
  (pad 3 thru_hole oval (at 5 0 270) (size 1.7 1.95) (drill 0.95) (layers *.Cu *.Mask) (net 14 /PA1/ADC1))
  (pad 2 thru_hole oval (at 2.5 0 270) (size 1.7 1.95) (drill 0.95) (layers *.Cu *.Mask) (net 2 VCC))
  (pad 1 thru_hole roundrect (at 0 0 270) (size 1.7 1.95) (drill 0.95) (layers *.Cu *.Mask) (roundrect_rratio 0.147059) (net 1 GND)))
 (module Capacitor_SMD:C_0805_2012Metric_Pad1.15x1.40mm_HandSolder (layer F.Cu) (at 95.25 57.15 90)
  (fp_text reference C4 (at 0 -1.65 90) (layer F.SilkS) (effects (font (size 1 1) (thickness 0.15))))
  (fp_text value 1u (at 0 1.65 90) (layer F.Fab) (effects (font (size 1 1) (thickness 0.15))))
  (pad 2 smd roundrect (at 1.025 0 90) (size 1.15 1.4) (layers F.Cu F.Paste F.Mask) (roundrect_rratio 0.217391) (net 1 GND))
  (pad 1 smd roundrect (at -1.025 0 90) (size 1.15 1.4) (layers F.Cu F.Paste F.Mask) (roundrect_rratio 0.217391) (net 2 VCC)))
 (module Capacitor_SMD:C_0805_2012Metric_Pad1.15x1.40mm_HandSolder (layer F.Cu) (at 154.94 95.25 270)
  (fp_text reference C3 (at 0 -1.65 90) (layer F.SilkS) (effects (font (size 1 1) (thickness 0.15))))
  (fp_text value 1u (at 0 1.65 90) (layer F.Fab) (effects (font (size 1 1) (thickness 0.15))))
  (pad 2 smd roundrect (at 1.025 0 270) (size 1.15 1.4) (layers F.Cu F.Paste F.Mask) (roundrect_rratio 0.217391) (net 1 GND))
  (pad 1 smd roundrect (at -1.025 0 270) (size 1.15 1.4) (layers F.Cu F.Paste F.Mask) (roundrect_rratio 0.217391) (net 45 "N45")))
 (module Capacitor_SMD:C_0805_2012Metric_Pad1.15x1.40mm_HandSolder (layer F.Cu) (at 160.02 83.82 90)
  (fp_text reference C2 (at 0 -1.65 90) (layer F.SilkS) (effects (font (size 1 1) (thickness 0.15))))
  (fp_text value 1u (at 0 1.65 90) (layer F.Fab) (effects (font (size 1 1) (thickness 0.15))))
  (pad 2 smd roundrect (at 1.025 0 90) (size 1.15 1.4) (layers F.Cu F.Paste F.Mask) (roundrect_rratio 0.217391) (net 1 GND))
  (pad 1 smd roundrect (at -1.025 0 90) (size 1.15 1.4) (layers F.Cu F.Paste F.Mask) (roundrect_rratio 0.217391) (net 19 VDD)))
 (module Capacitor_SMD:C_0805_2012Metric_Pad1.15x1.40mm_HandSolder (layer F.Cu) (at 149.86 76.2 270)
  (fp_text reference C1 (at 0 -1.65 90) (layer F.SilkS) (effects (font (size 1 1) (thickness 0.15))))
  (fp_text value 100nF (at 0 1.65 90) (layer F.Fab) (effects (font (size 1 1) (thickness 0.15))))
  (pad 2 smd roundrect (at 1.025 0 270) (size 1.15 1.4) (layers F.Cu F.Paste F.Mask) (roundrect_rratio 0.217391) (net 1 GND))
  (pad 1 smd roundrect (at -1.025 0 270) (size 1.15 1.4) (layers F.Cu F.Paste F.Mask) (roundrect_rratio 0.217391) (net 15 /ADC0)))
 (gr_line (start 187.96 100.33) (end 90.17 100.33) (layer Edge.Cuts) (width 0.1))
 (gr_line (start 187.96 50.8) (end 187.96 100.33) (layer Edge.Cuts) (width 0.1))
 (gr_line (start 90.17 50.8) (end 187.96 50.8) (layer Edge.Cuts) (width 0.1))
 (gr_line (start 90.17 100.33) (end 90.17 50.8) (layer Edge.Cuts) (width 0.1))
 (segment (start 105.41 68.58) (end 102.87 68.58) (width 0.25) (layer F.Cu) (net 1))
 (segment (start 102.87 68.58) (end 96.52 68.58) (width 0.25) (layer F.Cu) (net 1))
 (segment (start 96.52 68.58) (end 93.98 71.12) (width 0.25) (layer F.Cu) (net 1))
 (segment (start 96.52 71.12) (end 96.52 71.08) (width 0.25) (layer F.Cu) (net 2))
 (segment (start 93.98 73.66) (end 96.52 71.12) (width 0.25) (layer F.Cu) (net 2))
 (segment (start 105.45 71.08) (end 107.95 68.58) (width 0.25) (layer F.Cu) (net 2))
 (segment (start 96.52 71.08) (end 105.45 71.08) (width 0.25) (layer F.Cu) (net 2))
 (segment (start 97.745 78.58) (end 97.905 78.74) (width 0.25) (layer F.Cu) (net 32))
 (segment (start 96.52 78.58) (end 97.745 78.58) (width 0.25) (layer F.Cu) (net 32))
 (segment (start 97.905 78.74) (end 111.76 78.74) (width 0.25) (layer F.Cu) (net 32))
 (segment (start 113.03 80.01) (end 113.03 83.82) (width 0.25) (layer F.Cu) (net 32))
 (segment (start 111.76 78.74) (end 113.03 80.01) (width 0.25) (layer F.Cu) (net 32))
 (segment (start 97.745 81.08) (end 97.945 81.28) (width 0.25) (layer F.Cu) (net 34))
 (segment (start 96.52 81.08) (end 97.745 81.08) (width 0.25) (layer F.Cu) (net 34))
 (segment (start 105.41 81.28) (end 106.68 82.55) (width 0.25) (layer F.Cu) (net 34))
 (segment (start 97.945 81.28) (end 105.41 81.28) (width 0.25) (layer F.Cu) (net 34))
 (segment (start 106.68 82.55) (end 107.95 83.82) (width 0.25) (layer F.Cu) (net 34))
 (segment (start 96.32 81.08) (end 96.52 81.08) (width 0.25) (layer F.Cu) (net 34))
 (segment (start 93.98 78.74) (end 96.32 81.08) (width 0.25) (layer F.Cu) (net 34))
 (segment (start 97.745 76.08) (end 97.865 76.2) (width 0.25) (layer F.Cu) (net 33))
 (segment (start 96.52 76.08) (end 97.745 76.08) (width 0.25) (layer F.Cu) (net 33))
 (segment (start 96.52 76.2) (end 110.49 76.2) (width 0.25) (layer F.Cu) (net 33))
 (via (at 110.49 76.2) (size 0.8) (drill 0.4) (layers F.Cu B.Cu) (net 33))
 (segment (start 110.49 76.2) (end 110.49 83.82) (width 0.25) (layer B.Cu) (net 33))
 (segment (start 93.74 83.58) (end 96.52 83.58) (width 0.25) (layer F.Cu) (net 35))
 (segment (start 91.44 81.28) (end 93.74 83.58) (width 0.25) (layer F.Cu) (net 35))
 (segment (start 93.98 76.2) (end 91.44 76.2) (width 0.25) (layer F.Cu) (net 35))
 (segment (start 91.44 76.2) (end 91.44 81.28) (width 0.25) (layer F.Cu) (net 35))
 (segment (start 97.745 83.58) (end 97.79 83.625) (width 0.25) (layer F.Cu) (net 35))
 (segment (start 96.52 83.58) (end 97.745 83.58) (width 0.25) (layer F.Cu) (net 35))
 (segment (start 97.79 83.625) (end 98.865 83.625) (width 0.25) (layer F.Cu) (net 35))
 (segment (start 98.865 83.625) (end 101.6 86.36) (width 0.25) (layer F.Cu) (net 35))
 (segment (start 102.87 86.36) (end 105.41 83.82) (width 0.25) (layer F.Cu) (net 35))
 (segment (start 101.6 86.36) (end 102.87 86.36) (width 0.25) (layer F.Cu) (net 35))
 (segment (start 96.52 73.66) (end 100.33 73.66) (width 0.25) (layer B.Cu) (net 36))
 (segment (start 102.87 76.2) (end 102.87 83.82) (width 0.25) (layer B.Cu) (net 36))
 (segment (start 100.33 73.66) (end 102.87 76.2) (width 0.25) (layer B.Cu) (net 36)))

